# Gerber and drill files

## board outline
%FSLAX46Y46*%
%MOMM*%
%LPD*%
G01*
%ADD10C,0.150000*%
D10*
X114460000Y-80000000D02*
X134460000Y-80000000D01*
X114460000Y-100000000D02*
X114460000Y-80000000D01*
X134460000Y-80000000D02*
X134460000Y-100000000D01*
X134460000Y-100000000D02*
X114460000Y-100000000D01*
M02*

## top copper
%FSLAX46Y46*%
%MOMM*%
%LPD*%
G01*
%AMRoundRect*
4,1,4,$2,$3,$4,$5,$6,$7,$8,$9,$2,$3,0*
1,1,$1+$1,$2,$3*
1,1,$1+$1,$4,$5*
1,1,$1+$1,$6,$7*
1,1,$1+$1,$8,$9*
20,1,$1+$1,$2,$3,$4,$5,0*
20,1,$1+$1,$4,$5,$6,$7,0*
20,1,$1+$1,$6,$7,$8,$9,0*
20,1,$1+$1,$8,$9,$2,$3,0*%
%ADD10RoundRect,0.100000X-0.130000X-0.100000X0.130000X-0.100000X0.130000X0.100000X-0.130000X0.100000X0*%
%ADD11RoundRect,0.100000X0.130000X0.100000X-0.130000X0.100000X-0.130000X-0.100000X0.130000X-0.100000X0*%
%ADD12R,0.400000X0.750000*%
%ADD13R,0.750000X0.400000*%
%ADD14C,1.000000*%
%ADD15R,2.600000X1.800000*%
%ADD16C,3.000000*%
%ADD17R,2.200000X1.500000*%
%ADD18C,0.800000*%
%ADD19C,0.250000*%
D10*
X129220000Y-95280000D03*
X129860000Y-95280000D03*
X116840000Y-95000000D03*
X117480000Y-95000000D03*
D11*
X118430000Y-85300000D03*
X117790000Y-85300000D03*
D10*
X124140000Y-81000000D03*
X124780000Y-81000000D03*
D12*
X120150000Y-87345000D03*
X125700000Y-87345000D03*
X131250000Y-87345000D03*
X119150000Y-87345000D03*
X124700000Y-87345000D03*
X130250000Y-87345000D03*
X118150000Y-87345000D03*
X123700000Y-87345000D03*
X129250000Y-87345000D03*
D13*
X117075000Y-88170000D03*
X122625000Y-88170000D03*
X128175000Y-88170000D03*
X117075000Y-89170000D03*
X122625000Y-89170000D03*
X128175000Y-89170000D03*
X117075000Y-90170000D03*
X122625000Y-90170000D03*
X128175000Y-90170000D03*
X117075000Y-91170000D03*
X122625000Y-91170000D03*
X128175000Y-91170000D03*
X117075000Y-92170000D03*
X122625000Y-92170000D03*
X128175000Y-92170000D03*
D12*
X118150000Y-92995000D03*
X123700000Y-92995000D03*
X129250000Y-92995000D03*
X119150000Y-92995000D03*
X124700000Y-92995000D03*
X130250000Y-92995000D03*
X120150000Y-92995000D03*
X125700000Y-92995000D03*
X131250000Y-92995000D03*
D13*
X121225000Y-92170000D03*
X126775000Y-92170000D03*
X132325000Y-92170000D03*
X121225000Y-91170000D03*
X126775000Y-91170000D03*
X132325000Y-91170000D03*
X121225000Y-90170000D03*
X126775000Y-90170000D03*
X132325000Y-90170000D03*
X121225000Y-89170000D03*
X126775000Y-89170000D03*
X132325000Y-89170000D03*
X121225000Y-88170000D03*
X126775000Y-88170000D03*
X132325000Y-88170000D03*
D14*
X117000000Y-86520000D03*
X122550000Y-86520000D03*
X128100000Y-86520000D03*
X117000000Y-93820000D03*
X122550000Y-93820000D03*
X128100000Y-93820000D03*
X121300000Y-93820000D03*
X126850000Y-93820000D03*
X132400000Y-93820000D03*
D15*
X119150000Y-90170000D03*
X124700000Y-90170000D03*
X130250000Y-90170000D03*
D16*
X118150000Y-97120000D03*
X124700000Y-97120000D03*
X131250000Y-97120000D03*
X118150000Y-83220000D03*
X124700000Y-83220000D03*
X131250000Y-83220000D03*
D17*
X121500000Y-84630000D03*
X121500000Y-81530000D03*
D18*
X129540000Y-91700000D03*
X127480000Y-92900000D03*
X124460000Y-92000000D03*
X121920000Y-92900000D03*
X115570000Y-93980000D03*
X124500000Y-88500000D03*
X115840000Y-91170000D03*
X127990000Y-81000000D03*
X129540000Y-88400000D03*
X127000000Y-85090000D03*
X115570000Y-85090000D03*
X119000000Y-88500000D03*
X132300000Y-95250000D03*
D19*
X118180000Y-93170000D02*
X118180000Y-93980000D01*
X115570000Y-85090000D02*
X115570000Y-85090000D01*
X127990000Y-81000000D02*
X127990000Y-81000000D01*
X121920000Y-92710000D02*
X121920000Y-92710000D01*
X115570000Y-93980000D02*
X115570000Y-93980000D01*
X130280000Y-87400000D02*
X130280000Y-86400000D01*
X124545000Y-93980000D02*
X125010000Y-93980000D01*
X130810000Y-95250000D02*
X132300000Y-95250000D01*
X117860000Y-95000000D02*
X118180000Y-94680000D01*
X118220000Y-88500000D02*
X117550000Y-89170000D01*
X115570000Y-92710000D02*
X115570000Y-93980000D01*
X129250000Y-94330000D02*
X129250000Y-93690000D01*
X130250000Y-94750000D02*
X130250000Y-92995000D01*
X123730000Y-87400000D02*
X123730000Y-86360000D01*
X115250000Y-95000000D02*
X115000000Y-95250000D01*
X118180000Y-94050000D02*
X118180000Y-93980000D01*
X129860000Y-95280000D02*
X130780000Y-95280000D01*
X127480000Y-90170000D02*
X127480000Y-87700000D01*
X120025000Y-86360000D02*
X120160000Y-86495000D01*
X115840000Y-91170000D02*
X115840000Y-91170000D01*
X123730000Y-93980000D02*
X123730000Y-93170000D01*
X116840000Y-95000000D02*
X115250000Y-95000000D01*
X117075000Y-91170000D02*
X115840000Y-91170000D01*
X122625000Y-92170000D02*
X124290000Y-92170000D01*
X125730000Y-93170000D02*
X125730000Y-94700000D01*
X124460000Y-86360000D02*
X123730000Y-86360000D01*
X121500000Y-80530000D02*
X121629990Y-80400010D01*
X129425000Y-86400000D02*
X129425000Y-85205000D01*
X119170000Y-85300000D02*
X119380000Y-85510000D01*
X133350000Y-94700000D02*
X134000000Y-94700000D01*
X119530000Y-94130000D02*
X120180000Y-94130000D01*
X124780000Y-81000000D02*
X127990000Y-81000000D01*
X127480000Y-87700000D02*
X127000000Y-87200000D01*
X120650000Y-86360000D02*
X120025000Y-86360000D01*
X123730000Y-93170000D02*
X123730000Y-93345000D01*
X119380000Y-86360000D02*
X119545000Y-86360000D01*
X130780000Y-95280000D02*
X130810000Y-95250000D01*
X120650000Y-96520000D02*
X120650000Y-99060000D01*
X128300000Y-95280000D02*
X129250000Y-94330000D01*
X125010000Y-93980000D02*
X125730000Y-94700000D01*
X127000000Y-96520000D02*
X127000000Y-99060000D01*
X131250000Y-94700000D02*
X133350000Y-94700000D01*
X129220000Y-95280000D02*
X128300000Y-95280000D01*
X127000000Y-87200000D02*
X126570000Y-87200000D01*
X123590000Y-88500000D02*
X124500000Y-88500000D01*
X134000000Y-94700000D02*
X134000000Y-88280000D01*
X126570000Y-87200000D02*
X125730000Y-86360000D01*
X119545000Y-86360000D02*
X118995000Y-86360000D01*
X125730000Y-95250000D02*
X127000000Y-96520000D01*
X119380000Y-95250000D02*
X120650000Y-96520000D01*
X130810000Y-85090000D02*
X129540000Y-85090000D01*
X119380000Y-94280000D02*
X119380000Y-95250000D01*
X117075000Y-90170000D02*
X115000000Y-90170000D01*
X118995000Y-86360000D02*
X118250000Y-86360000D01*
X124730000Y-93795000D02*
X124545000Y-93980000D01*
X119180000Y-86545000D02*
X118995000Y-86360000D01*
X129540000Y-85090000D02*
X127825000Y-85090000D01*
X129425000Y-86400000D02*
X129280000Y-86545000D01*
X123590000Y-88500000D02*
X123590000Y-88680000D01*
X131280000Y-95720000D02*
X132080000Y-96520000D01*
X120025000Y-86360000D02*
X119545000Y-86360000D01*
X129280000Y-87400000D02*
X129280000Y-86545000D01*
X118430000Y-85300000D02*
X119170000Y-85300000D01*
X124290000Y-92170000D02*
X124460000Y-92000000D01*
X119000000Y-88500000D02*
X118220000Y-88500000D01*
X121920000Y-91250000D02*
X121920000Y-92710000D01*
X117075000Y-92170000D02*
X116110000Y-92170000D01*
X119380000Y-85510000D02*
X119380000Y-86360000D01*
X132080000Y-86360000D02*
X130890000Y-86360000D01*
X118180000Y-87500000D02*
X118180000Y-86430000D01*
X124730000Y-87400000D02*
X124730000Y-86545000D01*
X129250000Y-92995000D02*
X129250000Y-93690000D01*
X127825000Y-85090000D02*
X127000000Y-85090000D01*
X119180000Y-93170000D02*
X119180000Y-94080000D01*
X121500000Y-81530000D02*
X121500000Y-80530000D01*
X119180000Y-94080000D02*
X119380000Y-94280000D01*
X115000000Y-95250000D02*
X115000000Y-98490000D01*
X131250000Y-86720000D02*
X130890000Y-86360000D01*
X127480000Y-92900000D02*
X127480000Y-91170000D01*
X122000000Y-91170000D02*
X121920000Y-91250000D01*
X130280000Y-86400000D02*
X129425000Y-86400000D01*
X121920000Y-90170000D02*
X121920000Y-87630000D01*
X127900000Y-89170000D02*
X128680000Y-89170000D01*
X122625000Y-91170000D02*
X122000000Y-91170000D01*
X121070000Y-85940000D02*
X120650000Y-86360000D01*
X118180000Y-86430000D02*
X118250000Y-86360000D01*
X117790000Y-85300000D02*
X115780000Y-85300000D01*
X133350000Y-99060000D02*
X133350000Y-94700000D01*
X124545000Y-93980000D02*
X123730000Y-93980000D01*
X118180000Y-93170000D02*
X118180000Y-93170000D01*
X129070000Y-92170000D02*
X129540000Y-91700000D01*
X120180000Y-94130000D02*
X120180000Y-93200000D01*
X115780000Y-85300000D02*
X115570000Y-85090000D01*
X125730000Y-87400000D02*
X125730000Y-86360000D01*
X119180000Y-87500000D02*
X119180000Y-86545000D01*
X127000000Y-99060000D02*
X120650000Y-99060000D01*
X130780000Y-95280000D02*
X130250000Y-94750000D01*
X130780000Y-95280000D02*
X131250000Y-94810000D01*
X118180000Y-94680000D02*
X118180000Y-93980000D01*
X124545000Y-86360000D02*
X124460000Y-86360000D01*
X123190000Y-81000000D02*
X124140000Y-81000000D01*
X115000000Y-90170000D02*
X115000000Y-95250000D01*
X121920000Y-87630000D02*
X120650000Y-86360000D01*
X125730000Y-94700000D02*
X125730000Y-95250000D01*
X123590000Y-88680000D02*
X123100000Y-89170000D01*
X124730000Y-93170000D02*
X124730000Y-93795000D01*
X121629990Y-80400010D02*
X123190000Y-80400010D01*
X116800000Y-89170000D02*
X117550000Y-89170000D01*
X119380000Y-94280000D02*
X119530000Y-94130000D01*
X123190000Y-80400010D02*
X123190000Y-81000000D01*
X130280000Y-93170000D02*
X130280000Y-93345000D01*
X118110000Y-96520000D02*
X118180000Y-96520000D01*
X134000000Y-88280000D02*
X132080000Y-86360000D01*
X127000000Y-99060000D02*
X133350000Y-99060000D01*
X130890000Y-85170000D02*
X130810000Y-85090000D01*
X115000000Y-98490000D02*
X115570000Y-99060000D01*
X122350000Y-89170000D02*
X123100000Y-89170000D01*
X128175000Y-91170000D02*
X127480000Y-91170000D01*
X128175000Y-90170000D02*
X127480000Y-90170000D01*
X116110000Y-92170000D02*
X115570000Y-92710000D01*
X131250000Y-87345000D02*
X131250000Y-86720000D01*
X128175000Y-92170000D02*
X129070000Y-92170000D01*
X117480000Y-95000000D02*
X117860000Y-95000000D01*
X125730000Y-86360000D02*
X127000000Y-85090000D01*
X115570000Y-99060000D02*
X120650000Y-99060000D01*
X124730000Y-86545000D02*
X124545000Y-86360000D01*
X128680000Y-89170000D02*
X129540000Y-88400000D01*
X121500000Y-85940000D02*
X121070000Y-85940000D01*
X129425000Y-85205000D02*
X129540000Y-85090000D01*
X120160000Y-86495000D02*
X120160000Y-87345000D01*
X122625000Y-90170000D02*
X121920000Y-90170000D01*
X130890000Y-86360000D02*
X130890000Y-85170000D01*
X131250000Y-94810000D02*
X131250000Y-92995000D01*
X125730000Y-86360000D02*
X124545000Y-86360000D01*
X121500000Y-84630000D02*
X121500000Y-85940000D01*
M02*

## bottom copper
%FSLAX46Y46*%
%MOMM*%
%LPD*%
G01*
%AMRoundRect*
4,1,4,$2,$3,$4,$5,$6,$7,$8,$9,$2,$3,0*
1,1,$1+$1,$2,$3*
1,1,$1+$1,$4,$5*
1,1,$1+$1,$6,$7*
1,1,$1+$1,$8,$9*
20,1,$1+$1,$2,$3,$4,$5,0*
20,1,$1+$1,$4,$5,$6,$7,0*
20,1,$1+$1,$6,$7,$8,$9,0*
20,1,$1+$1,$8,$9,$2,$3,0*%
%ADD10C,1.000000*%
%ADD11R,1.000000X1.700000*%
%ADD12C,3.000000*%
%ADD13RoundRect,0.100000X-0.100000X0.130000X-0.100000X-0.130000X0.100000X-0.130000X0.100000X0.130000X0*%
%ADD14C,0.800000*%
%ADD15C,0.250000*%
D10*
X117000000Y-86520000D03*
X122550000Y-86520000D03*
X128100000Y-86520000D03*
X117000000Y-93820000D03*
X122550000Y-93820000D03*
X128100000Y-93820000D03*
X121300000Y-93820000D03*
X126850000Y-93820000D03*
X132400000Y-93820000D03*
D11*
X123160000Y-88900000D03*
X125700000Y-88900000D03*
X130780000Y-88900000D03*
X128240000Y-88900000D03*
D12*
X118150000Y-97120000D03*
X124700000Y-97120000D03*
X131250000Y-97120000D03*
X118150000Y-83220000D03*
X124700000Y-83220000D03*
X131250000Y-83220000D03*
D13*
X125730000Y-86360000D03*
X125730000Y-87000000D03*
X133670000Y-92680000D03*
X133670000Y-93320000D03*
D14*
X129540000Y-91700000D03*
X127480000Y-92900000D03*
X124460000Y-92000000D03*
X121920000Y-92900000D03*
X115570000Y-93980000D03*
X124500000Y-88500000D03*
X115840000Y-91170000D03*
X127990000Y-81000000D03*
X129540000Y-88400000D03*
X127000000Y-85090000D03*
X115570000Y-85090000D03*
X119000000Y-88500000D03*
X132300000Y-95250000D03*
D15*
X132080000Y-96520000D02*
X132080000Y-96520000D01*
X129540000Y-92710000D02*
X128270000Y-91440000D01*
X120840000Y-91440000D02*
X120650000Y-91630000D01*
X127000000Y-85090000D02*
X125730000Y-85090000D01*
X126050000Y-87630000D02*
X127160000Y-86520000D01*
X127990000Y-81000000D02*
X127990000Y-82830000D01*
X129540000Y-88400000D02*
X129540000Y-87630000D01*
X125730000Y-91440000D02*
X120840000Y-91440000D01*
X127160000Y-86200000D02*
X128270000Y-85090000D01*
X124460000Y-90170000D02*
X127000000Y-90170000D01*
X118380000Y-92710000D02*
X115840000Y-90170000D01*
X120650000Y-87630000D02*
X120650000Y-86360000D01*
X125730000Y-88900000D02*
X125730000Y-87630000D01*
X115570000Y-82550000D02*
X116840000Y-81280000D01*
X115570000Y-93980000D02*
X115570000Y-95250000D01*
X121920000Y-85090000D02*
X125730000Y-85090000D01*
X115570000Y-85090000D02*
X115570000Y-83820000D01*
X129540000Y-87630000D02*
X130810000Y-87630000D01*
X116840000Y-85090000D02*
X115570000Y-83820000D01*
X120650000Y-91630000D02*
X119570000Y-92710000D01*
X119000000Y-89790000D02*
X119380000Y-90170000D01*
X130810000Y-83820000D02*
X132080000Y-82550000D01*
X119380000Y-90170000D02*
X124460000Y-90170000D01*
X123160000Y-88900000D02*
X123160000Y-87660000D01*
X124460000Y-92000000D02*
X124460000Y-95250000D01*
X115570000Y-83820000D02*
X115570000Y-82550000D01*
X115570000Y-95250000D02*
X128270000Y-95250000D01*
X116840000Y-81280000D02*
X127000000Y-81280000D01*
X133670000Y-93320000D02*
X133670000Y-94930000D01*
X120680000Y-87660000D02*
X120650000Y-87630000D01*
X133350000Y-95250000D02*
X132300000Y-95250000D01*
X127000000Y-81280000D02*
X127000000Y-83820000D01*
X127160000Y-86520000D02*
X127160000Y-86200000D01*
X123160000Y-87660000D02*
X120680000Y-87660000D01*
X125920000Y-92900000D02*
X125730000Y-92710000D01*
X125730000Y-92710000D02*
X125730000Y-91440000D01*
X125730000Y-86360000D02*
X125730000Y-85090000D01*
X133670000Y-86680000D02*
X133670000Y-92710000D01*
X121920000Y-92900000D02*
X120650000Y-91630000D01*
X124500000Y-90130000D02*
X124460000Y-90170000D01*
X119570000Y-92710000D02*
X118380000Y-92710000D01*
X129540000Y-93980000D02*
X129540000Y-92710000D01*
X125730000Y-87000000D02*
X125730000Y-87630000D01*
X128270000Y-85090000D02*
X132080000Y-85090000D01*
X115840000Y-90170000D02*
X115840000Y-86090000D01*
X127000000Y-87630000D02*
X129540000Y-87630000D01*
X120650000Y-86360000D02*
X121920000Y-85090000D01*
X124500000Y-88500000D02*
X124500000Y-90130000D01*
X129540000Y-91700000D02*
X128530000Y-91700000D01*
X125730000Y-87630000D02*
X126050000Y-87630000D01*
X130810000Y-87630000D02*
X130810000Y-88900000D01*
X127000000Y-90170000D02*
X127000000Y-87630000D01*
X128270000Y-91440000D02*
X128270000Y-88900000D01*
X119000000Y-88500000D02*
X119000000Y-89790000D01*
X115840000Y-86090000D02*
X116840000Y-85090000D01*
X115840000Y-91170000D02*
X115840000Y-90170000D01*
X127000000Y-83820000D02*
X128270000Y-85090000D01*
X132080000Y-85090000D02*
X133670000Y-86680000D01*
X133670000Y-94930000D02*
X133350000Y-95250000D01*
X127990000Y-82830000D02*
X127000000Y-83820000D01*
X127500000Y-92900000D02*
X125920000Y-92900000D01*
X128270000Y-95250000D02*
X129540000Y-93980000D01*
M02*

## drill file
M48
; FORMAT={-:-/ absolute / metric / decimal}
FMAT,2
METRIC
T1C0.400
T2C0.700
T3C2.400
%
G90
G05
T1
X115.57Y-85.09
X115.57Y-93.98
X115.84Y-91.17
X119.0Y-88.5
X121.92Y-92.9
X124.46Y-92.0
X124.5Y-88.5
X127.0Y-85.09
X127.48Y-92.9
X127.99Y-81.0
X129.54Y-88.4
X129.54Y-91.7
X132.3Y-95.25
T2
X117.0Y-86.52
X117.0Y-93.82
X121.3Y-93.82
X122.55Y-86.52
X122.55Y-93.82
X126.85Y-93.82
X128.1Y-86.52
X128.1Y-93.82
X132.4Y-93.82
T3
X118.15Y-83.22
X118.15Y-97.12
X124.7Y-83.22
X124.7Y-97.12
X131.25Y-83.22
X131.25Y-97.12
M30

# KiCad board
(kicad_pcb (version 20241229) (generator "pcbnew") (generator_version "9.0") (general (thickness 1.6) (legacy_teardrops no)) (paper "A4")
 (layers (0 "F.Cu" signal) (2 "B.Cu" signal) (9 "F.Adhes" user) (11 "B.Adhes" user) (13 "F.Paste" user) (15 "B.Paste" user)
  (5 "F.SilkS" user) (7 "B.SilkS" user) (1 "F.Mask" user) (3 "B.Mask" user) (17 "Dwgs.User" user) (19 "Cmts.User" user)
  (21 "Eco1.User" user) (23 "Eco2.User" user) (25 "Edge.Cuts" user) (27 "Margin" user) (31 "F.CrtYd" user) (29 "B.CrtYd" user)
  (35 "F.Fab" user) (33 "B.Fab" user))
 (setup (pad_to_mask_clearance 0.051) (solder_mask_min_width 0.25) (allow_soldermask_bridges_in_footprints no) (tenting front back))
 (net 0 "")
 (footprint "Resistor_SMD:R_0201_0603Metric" (layer "F.Cu") (at 129.54 95.28)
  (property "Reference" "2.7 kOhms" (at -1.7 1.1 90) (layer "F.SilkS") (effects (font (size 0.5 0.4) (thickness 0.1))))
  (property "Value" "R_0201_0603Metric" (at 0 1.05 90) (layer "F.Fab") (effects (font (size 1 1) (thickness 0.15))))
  (pad "" smd roundrect (at -0.345 0) (size 0.318 0.36) (layers "F.Paste") (roundrect_rratio 0.25))
  (pad "" smd roundrect (at 0.345 0) (size 0.318 0.36) (layers "F.Paste") (roundrect_rratio 0.25))
  (pad "1" smd roundrect (at -0.32 0) (size 0.46 0.4) (layers "F.Cu" "F.Mask") (roundrect_rratio 0.25))
  (pad "2" smd roundrect (at 0.32 0) (size 0.46 0.4) (layers "F.Cu" "F.Mask") (roundrect_rratio 0.25)))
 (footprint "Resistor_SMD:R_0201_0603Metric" (layer "F.Cu") (at 117.16 95)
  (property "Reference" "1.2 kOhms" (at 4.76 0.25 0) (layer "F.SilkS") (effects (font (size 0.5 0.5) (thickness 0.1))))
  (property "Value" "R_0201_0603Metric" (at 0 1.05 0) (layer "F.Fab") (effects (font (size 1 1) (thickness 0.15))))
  (pad "" smd roundrect (at -0.345 0) (size 0.318 0.36) (layers "F.Paste") (roundrect_rratio 0.25))
  (pad "" smd roundrect (at 0.345 0) (size 0.318 0.36) (layers "F.Paste") (roundrect_rratio 0.25))
  (pad "1" smd roundrect (at -0.32 0) (size 0.46 0.4) (layers "F.Cu" "F.Mask") (roundrect_rratio 0.25))
  (pad "2" smd roundrect (at 0.32 0) (size 0.46 0.4) (layers "F.Cu" "F.Mask") (roundrect_rratio 0.25)))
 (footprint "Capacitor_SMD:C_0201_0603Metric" (layer "F.Cu") (at 118.11 85.3 180)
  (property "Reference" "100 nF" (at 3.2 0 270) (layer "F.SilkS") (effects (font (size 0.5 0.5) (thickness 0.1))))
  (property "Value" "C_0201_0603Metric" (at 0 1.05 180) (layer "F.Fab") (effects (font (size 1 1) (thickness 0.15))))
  (pad "" smd roundrect (at -0.345 0 180) (size 0.318 0.36) (layers "F.Paste") (roundrect_rratio 0.25))
  (pad "" smd roundrect (at 0.345 0 180) (size 0.318 0.36) (layers "F.Paste") (roundrect_rratio 0.25))
  (pad "1" smd roundrect (at -0.32 0 180) (size 0.46 0.4) (layers "F.Cu" "F.Mask") (roundrect_rratio 0.25))
  (pad "2" smd roundrect (at 0.32 0 180) (size 0.46 0.4) (layers "F.Cu" "F.Mask") (roundrect_rratio 0.25)))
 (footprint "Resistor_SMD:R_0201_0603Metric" (layer "F.Cu") (at 124.46 81)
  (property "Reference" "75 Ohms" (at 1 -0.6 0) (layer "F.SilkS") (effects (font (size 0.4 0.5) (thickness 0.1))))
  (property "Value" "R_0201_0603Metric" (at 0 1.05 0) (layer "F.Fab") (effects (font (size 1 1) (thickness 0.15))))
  (pad "" smd roundrect (at -0.345 0) (size 0.318 0.36) (layers "F.Paste") (roundrect_rratio 0.25))
  (pad "" smd roundrect (at 0.345 0) (size 0.318 0.36) (layers "F.Paste") (roundrect_rratio 0.25))
  (pad "1" smd roundrect (at -0.32 0) (size 0.46 0.4) (layers "F.Cu" "F.Mask") (roundrect_rratio 0.25))
  (pad "2" smd roundrect (at 0.32 0) (size 0.46 0.4) (layers "F.Cu" "F.Mask") (roundrect_rratio 0.25)))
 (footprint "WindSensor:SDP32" (layer "F.Cu") (at 124.7 90.17)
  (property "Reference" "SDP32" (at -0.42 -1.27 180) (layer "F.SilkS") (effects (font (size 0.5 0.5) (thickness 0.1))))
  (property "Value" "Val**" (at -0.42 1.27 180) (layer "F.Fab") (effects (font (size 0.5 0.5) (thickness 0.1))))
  (pad "1" smd rect (at -4.55 -2.825 270) (size 0.75 0.4) (layers "F.Cu" "F.Mask" "F.Paste"))
  (pad "1" smd rect (at 1 -2.825 270) (size 0.75 0.4) (layers "F.Cu" "F.Mask" "F.Paste"))
  (pad "1" smd rect (at 6.55 -2.825 270) (size 0.75 0.4) (layers "F.Cu" "F.Mask" "F.Paste"))
  (pad "2" smd rect (at -5.55 -2.825 270) (size 0.75 0.4) (layers "F.Cu" "F.Mask" "F.Paste"))
  (pad "2" smd rect (at 0 -2.825 270) (size 0.75 0.4) (layers "F.Cu" "F.Mask" "F.Paste"))
  (pad "2" smd rect (at 5.55 -2.825 270) (size 0.75 0.4) (layers "F.Cu" "F.Mask" "F.Paste"))
  (pad "3" smd rect (at -6.55 -2.825 270) (size 0.75 0.4) (layers "F.Cu" "F.Mask" "F.Paste"))
  (pad "3" smd rect (at -1 -2.825 270) (size 0.75 0.4) (layers "F.Cu" "F.Mask" "F.Paste"))
  (pad "3" smd rect (at 4.55 -2.825 270) (size 0.75 0.4) (layers "F.Cu" "F.Mask" "F.Paste"))
  (pad "4" smd rect (at -7.625 -2 270) (size 0.4 0.75) (layers "F.Cu" "F.Mask" "F.Paste"))
  (pad "4" smd rect (at -2.075 -2 270) (size 0.4 0.75) (layers "F.Cu" "F.Mask" "F.Paste"))
  (pad "4" smd rect (at 3.475 -2 270) (size 0.4 0.75) (layers "F.Cu" "F.Mask" "F.Paste"))
  (pad "5" smd rect (at -7.625 -1 270) (size 0.4 0.75) (layers "F.Cu" "F.Mask" "F.Paste"))
  (pad "5" smd rect (at -2.075 -1 270) (size 0.4 0.75) (layers "F.Cu" "F.Mask" "F.Paste"))
  (pad "5" smd rect (at 3.475 -1 270) (size 0.4 0.75) (layers "F.Cu" "F.Mask" "F.Paste"))
  (pad "6" smd rect (at -7.625 0 270) (size 0.4 0.75) (layers "F.Cu" "F.Mask" "F.Paste"))
  (pad "6" smd rect (at -2.075 0 270) (size 0.4 0.75) (layers "F.Cu" "F.Mask" "F.Paste"))
  (pad "6" smd rect (at 3.475 0 270) (size 0.4 0.75) (layers "F.Cu" "F.Mask" "F.Paste"))
  (pad "7" smd rect (at -7.625 1 270) (size 0.4 0.75) (layers "F.Cu" "F.Mask" "F.Paste"))
  (pad "7" smd rect (at -2.075 1 270) (size 0.4 0.75) (layers "F.Cu" "F.Mask" "F.Paste"))
  (pad "7" smd rect (at 3.475 1 270) (size 0.4 0.75) (layers "F.Cu" "F.Mask" "F.Paste"))
  (pad "8" smd rect (at -7.625 2 270) (size 0.4 0.75) (layers "F.Cu" "F.Mask" "F.Paste"))
  (pad "8" smd rect (at -2.075 2 270) (size 0.4 0.75) (layers "F.Cu" "F.Mask" "F.Paste"))
  (pad "8" smd rect (at 3.475 2 270) (size 0.4 0.75) (layers "F.Cu" "F.Mask" "F.Paste"))
  (pad "9" smd rect (at -6.55 2.825 270) (size 0.75 0.4) (layers "F.Cu" "F.Mask" "F.Paste"))
  (pad "9" smd rect (at -1 2.825 270) (size 0.75 0.4) (layers "F.Cu" "F.Mask" "F.Paste"))
  (pad "9" smd rect (at 4.55 2.825 270) (size 0.75 0.4) (layers "F.Cu" "F.Mask" "F.Paste"))
  (pad "10" smd rect (at -5.55 2.825 270) (size 0.75 0.4) (layers "F.Cu" "F.Mask" "F.Paste"))
  (pad "10" smd rect (at 0 2.825 270) (size 0.75 0.4) (layers "F.Cu" "F.Mask" "F.Paste"))
  (pad "10" smd rect (at 5.55 2.825 270) (size 0.75 0.4) (layers "F.Cu" "F.Mask" "F.Paste"))
  (pad "11" smd rect (at -4.55 2.825 270) (size 0.75 0.4) (layers "F.Cu" "F.Mask" "F.Paste"))
  (pad "11" smd rect (at 1 2.825 270) (size 0.75 0.4) (layers "F.Cu" "F.Mask" "F.Paste"))
  (pad "11" smd rect (at 6.55 2.825 270) (size 0.75 0.4) (layers "F.Cu" "F.Mask" "F.Paste"))
  (pad "12" smd rect (at -3.475 2 270) (size 0.4 0.75) (layers "F.Cu" "F.Mask" "F.Paste"))
  (pad "12" smd rect (at 2.075 2 270) (size 0.4 0.75) (layers "F.Cu" "F.Mask" "F.Paste"))
  (pad "12" smd rect (at 7.625 2 270) (size 0.4 0.75) (layers "F.Cu" "F.Mask" "F.Paste"))
  (pad "13" smd rect (at -3.475 1 270) (size 0.4 0.75) (layers "F.Cu" "F.Mask" "F.Paste"))
  (pad "13" smd rect (at 2.075 1 270) (size 0.4 0.75) (layers "F.Cu" "F.Mask" "F.Paste"))
  (pad "13" smd rect (at 7.625 1 270) (size 0.4 0.75) (layers "F.Cu" "F.Mask" "F.Paste"))
  (pad "14" smd rect (at -3.475 0 270) (size 0.4 0.75) (layers "F.Cu" "F.Mask" "F.Paste"))
  (pad "14" smd rect (at 2.075 0 270) (size 0.4 0.75) (layers "F.Cu" "F.Mask" "F.Paste"))
  (pad "14" smd rect (at 7.625 0 270) (size 0.4 0.75) (layers "F.Cu" "F.Mask" "F.Paste"))
  (pad "15" smd rect (at -3.475 -1 270) (size 0.4 0.75) (layers "F.Cu" "F.Mask" "F.Paste"))
  (pad "15" smd rect (at 2.075 -1 270) (size 0.4 0.75) (layers "F.Cu" "F.Mask" "F.Paste"))
  (pad "15" smd rect (at 7.625 -1 270) (size 0.4 0.75) (layers "F.Cu" "F.Mask" "F.Paste"))
  (pad "16" smd rect (at -3.475 -2 270) (size 0.4 0.75) (layers "F.Cu" "F.Mask" "F.Paste"))
  (pad "16" smd rect (at 2.075 -2 270) (size 0.4 0.75) (layers "F.Cu" "F.Mask" "F.Paste"))
  (pad "16" smd rect (at 7.625 -2 270) (size 0.4 0.75) (layers "F.Cu" "F.Mask" "F.Paste"))
  (pad "17" thru_hole circle (at -7.7 -3.65 270) (size 1 1) (drill 0.7) (layers "*.Cu" "*.Mask") (remove_unused_layers no))
  (pad "17" thru_hole circle (at -2.15 -3.65 270) (size 1 1) (drill 0.7) (layers "*.Cu" "*.Mask") (remove_unused_layers no))
  (pad "17" thru_hole circle (at 3.4 -3.65 270) (size 1 1) (drill 0.7) (layers "*.Cu" "*.Mask") (remove_unused_layers no))
  (pad "18" thru_hole circle (at -7.7 3.65 270) (size 1 1) (drill 0.7) (layers "*.Cu" "*.Mask") (remove_unused_layers no))
  (pad "18" thru_hole circle (at -2.15 3.65 270) (size 1 1) (drill 0.7) (layers "*.Cu" "*.Mask") (remove_unused_layers no))
  (pad "18" thru_hole circle (at 3.4 3.65 270) (size 1 1) (drill 0.7) (layers "*.Cu" "*.Mask") (remove_unused_layers no))
  (pad "19" thru_hole circle (at -3.4 3.65 270) (size 1 1) (drill 0.7) (layers "*.Cu" "*.Mask") (remove_unused_layers no))
  (pad "19" thru_hole circle (at 2.15 3.65 270) (size 1 1) (drill 0.7) (layers "*.Cu" "*.Mask") (remove_unused_layers no))
  (pad "19" thru_hole circle (at 7.7 3.65 270) (size 1 1) (drill 0.7) (layers "*.Cu" "*.Mask") (remove_unused_layers no))
  (pad "20" smd rect (at -5.55 0 270) (size 1.8 2.6) (layers "F.Cu" "F.Mask" "F.Paste"))
  (pad "20" smd rect (at 0 0 270) (size 1.8 2.6) (layers "F.Cu" "F.Mask" "F.Paste"))
  (pad "20" smd rect (at 5.55 0 270) (size 1.8 2.6) (layers "F.Cu" "F.Mask" "F.Paste"))
  (pad "21" smd rect (at -1.54 -1.27) (size 1 1.7) (layers "B.Cu" "B.Mask" "B.Paste"))
  (pad "22" smd rect (at 1 -1.27) (size 1 1.7) (layers "B.Cu" "B.Mask" "B.Paste"))
  (pad "23" smd rect (at 6.08 -1.27) (size 1 1.7) (layers "B.Cu" "B.Mask" "B.Paste"))
  (pad "24" smd rect (at 3.54 -1.27) (size 1 1.7) (layers "B.Cu" "B.Mask" "B.Paste"))
  (pad "25" thru_hole circle (at -6.55 6.95) (size 3 3) (drill 2.4) (layers "*.Cu" "*.Mask") (remove_unused_layers no))
  (pad "26" thru_hole circle (at 0 6.95) (size 3 3) (drill 2.4) (layers "*.Cu" "*.Mask") (remove_unused_layers no))
  (pad "27" thru_hole circle (at 6.55 6.95) (size 3 3) (drill 2.4) (layers "*.Cu" "*.Mask") (remove_unused_layers no))
  (pad "28" thru_hole circle (at -6.55 -6.95) (size 3 3) (drill 2.4) (layers "*.Cu" "*.Mask") (remove_unused_layers no))
  (pad "29" thru_hole circle (at 0 -6.95) (size 3 3) (drill 2.4) (layers "*.Cu" "*.Mask") (remove_unused_layers no))
  (pad "30" thru_hole circle (at 6.55 -6.95) (size 3 3) (drill 2.4) (layers "*.Cu" "*.Mask") (remove_unused_layers no)))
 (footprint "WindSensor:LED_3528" (layer "F.Cu") (at 121.5 82.8 -90)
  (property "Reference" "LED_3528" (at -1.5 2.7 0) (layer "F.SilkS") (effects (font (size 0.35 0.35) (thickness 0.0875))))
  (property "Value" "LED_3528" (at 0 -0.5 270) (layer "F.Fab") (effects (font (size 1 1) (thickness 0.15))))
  (pad "1" smd rect (at 1.83 0 270) (size 1.5 2.2) (layers "F.Cu" "F.Mask" "F.Paste"))
  (pad "2" smd rect (at -1.27 0 270) (size 1.5 2.2) (layers "F.Cu" "F.Mask" "F.Paste")))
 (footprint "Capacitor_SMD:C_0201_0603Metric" (layer "B.Cu") (at 125.73 86.68 -90)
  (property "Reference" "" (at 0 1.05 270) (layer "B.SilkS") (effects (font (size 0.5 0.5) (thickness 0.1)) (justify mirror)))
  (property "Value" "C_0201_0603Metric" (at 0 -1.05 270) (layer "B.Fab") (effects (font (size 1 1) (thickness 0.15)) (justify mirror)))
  (pad "" smd roundrect (at -0.345 0 270) (size 0.318 0.36) (layers "B.Paste") (roundrect_rratio 0.25))
  (pad "" smd roundrect (at 0.345 0 270) (size 0.318 0.36) (layers "B.Paste") (roundrect_rratio 0.25))
  (pad "1" smd roundrect (at -0.32 0 270) (size 0.46 0.4) (layers "B.Cu" "B.Mask") (roundrect_rratio 0.25))
  (pad "2" smd roundrect (at 0.32 0 270) (size 0.46 0.4) (layers "B.Cu" "B.Mask") (roundrect_rratio 0.25)))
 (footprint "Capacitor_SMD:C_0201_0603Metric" (layer "B.Cu") (at 133.67 93 -90)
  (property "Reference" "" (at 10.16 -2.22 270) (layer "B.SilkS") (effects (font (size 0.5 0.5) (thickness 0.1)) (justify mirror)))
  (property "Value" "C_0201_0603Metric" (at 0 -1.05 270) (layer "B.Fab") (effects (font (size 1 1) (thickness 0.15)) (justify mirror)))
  (pad "" smd roundrect (at -0.345 0 270) (size 0.318 0.36) (layers "B.Paste") (roundrect_rratio 0.25))
  (pad "" smd roundrect (at 0.345 0 270) (size 0.318 0.36) (layers "B.Paste") (roundrect_rratio 0.25))
  (pad "1" smd roundrect (at -0.32 0 270) (size 0.46 0.4) (layers "B.Cu" "B.Mask") (roundrect_rratio 0.25))
  (pad "2" smd roundrect (at 0.32 0 270) (size 0.46 0.4) (layers "B.Cu" "B.Mask") (roundrect_rratio 0.25)))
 (gr_line (start 114.46 80) (end 134.46 80) (stroke (width 0.15) (type solid)) (layer "Edge.Cuts"))
 (gr_line (start 114.46 100) (end 114.46 80) (stroke (width 0.15) (type solid)) (layer "Edge.Cuts"))
 (gr_line (start 134.46 80) (end 134.46 100) (stroke (width 0.15) (type solid)) (layer "Edge.Cuts"))
 (gr_line (start 134.46 100) (end 114.46 100) (stroke (width 0.15) (type solid)) (layer "Edge.Cuts"))
 (segment (start 118.18 93.17) (end 118.18 93.98) (width 0.25) (layer "F.Cu") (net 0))
 (segment (start 115.57 85.09) (end 115.57 85.09) (width 0.25) (layer "F.Cu") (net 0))
 (segment (start 127.99 81) (end 127.99 81) (width 0.25) (layer "F.Cu") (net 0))
 (segment (start 121.92 92.71) (end 121.92 92.71) (width 0.25) (layer "F.Cu") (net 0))
 (segment (start 115.57 93.98) (end 115.57 93.98) (width 0.25) (layer "F.Cu") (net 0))
 (segment (start 130.28 87.4) (end 130.28 86.4) (width 0.25) (layer "F.Cu") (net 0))
 (segment (start 124.545 93.98) (end 125.01 93.98) (width 0.25) (layer "F.Cu") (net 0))
 (segment (start 130.81 95.25) (end 132.3 95.25) (width 0.25) (layer "F.Cu") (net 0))
 (segment (start 117.86 95) (end 118.18 94.68) (width 0.25) (layer "F.Cu") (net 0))
 (segment (start 118.22 88.5) (end 117.55 89.17) (width 0.25) (layer "F.Cu") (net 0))
 (segment (start 115.57 92.71) (end 115.57 93.98) (width 0.25) (layer "F.Cu") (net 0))
 (segment (start 129.25 94.33) (end 129.25 93.69) (width 0.25) (layer "F.Cu") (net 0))
 (segment (start 130.25 94.75) (end 130.25 92.995) (width 0.25) (layer "F.Cu") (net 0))
 (segment (start 123.73 87.4) (end 123.73 86.36) (width 0.25) (layer "F.Cu") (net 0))
 (segment (start 115.25 95) (end 115 95.25) (width 0.25) (layer "F.Cu") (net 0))
 (segment (start 118.18 94.05) (end 118.18 93.98) (width 0.25) (layer "F.Cu") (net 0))
 (segment (start 129.86 95.28) (end 130.78 95.28) (width 0.25) (layer "F.Cu") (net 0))
 (segment (start 127.48 90.17) (end 127.48 87.7) (width 0.25) (layer "F.Cu") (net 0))
 (segment (start 120.025 86.36) (end 120.16 86.495) (width 0.25) (layer "F.Cu") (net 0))
 (segment (start 115.84 91.17) (end 115.84 91.17) (width 0.25) (layer "F.Cu") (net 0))
 (segment (start 123.73 93.98) (end 123.73 93.17) (width 0.25) (layer "F.Cu") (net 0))
 (segment (start 116.84 95) (end 115.25 95) (width 0.25) (layer "F.Cu") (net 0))
 (segment (start 117.075 91.17) (end 115.84 91.17) (width 0.25) (layer "F.Cu") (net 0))
 (segment (start 122.625 92.17) (end 124.29 92.17) (width 0.25) (layer "F.Cu") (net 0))
 (segment (start 125.73 93.17) (end 125.73 94.7) (width 0.25) (layer "F.Cu") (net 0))
 (segment (start 124.46 86.36) (end 123.73 86.36) (width 0.25) (layer "F.Cu") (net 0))
 (segment (start 121.5 80.53) (end 121.62999 80.40001) (width 0.25) (layer "F.Cu") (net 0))
 (segment (start 129.425 86.4) (end 129.425 85.205) (width 0.25) (layer "F.Cu") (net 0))
 (segment (start 119.17 85.3) (end 119.38 85.51) (width 0.25) (layer "F.Cu") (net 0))
 (segment (start 133.35 94.7) (end 134 94.7) (width 0.25) (layer "F.Cu") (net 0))
 (segment (start 119.53 94.13) (end 120.18 94.13) (width 0.25) (layer "F.Cu") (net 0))
 (segment (start 124.78 81) (end 127.99 81) (width 0.25) (layer "F.Cu") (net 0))
 (segment (start 127.48 87.7) (end 127 87.2) (width 0.25) (layer "F.Cu") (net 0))
 (segment (start 120.65 86.36) (end 120.025 86.36) (width 0.25) (layer "F.Cu") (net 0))
 (segment (start 123.73 93.17) (end 123.73 93.345) (width 0.25) (layer "F.Cu") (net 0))
 (segment (start 119.38 86.36) (end 119.545 86.36) (width 0.25) (layer "F.Cu") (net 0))
 (segment (start 130.78 95.28) (end 130.81 95.25) (width 0.25) (layer "F.Cu") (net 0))
 (segment (start 120.65 96.52) (end 120.65 99.06) (width 0.25) (layer "F.Cu") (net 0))
 (segment (start 128.3 95.28) (end 129.25 94.33) (width 0.25) (layer "F.Cu") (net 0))
 (segment (start 125.01 93.98) (end 125.73 94.7) (width 0.25) (layer "F.Cu") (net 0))
 (segment (start 127 96.52) (end 127 99.06) (width 0.25) (layer "F.Cu") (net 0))
 (segment (start 131.25 94.7) (end 133.35 94.7) (width 0.25) (layer "F.Cu") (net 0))
 (segment (start 129.22 95.28) (end 128.3 95.28) (width 0.25) (layer "F.Cu") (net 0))
 (segment (start 127 87.2) (end 126.57 87.2) (width 0.25) (layer "F.Cu") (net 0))
 (segment (start 123.59 88.5) (end 124.5 88.5) (width 0.25) (layer "F.Cu") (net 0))
 (segment (start 134 94.7) (end 134 88.28) (width 0.25) (layer "F.Cu") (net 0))
 (segment (start 126.57 87.2) (end 125.73 86.36) (width 0.25) (layer "F.Cu") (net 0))
 (segment (start 119.545 86.36) (end 118.995 86.36) (width 0.25) (layer "F.Cu") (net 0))
 (segment (start 125.73 95.25) (end 127 96.52) (width 0.25) (layer "F.Cu") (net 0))
 (segment (start 119.38 95.25) (end 120.65 96.52) (width 0.25) (layer "F.Cu") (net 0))
 (segment (start 130.81 85.09) (end 129.54 85.09) (width 0.25) (layer "F.Cu") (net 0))
 (segment (start 119.38 94.28) (end 119.38 95.25) (width 0.25) (layer "F.Cu") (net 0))
 (segment (start 117.075 90.17) (end 115 90.17) (width 0.25) (layer "F.Cu") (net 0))
 (segment (start 118.995 86.36) (end 118.25 86.36) (width 0.25) (layer "F.Cu") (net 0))
 (segment (start 124.73 93.795) (end 124.545 93.98) (width 0.25) (layer "F.Cu") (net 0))
 (segment (start 119.18 86.545) (end 118.995 86.36) (width 0.25) (layer "F.Cu") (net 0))
 (segment (start 129.54 85.09) (end 127.825 85.09) (width 0.25) (layer "F.Cu") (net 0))
 (segment (start 129.425 86.4) (end 129.28 86.545) (width 0.25) (layer "F.Cu") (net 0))
 (segment (start 123.59 88.5) (end 123.59 88.68) (width 0.25) (layer "F.Cu") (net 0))
 (segment (start 131.28 95.72) (end 132.08 96.52) (width 0.25) (layer "F.Cu") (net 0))
 (segment (start 120.025 86.36) (end 119.545 86.36) (width 0.25) (layer "F.Cu") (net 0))
 (segment (start 129.28 87.4) (end 129.28 86.545) (width 0.25) (layer "F.Cu") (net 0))
 (segment (start 118.43 85.3) (end 119.17 85.3) (width 0.25) (layer "F.Cu") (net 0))
 (segment (start 124.29 92.17) (end 124.46 92) (width 0.25) (layer "F.Cu") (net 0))
 (segment (start 119 88.5) (end 118.22 88.5) (width 0.25) (layer "F.Cu") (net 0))
 (segment (start 121.92 91.25) (end 121.92 92.71) (width 0.25) (layer "F.Cu") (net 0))
 (segment (start 117.075 92.17) (end 116.11 92.17) (width 0.25) (layer "F.Cu") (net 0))
 (segment (start 119.38 85.51) (end 119.38 86.36) (width 0.25) (layer "F.Cu") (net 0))
 (segment (start 132.08 86.36) (end 130.89 86.36) (width 0.25) (layer "F.Cu") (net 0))
 (segment (start 118.18 87.5) (end 118.18 86.43) (width 0.25) (layer "F.Cu") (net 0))
 (segment (start 124.73 87.4) (end 124.73 86.545) (width 0.25) (layer "F.Cu") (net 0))
 (segment (start 129.25 92.995) (end 129.25 93.69) (width 0.25) (layer "F.Cu") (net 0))
 (segment (start 127.825 85.09) (end 127 85.09) (width 0.25) (layer "F.Cu") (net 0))
 (segment (start 119.18 93.17) (end 119.18 94.08) (width 0.25) (layer "F.Cu") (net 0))
 (segment (start 121.5 81.53) (end 121.5 80.53) (width 0.25) (layer "F.Cu") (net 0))
 (segment (start 119.18 94.08) (end 119.38 94.28) (width 0.25) (layer "F.Cu") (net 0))
 (segment (start 115 95.25) (end 115 98.49) (width 0.25) (layer "F.Cu") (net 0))
 (segment (start 131.25 86.72) (end 130.89 86.36) (width 0.25) (layer "F.Cu") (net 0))
 (segment (start 127.48 92.9) (end 127.48 91.17) (width 0.25) (layer "F.Cu") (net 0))
 (segment (start 122 91.17) (end 121.92 91.25) (width 0.25) (layer "F.Cu") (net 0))
 (segment (start 130.28 86.4) (end 129.425 86.4) (width 0.25) (layer "F.Cu") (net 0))
 (segment (start 121.92 90.17) (end 121.92 87.63) (width 0.25) (layer "F.Cu") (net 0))
 (segment (start 127.9 89.17) (end 128.68 89.17) (width 0.25) (layer "F.Cu") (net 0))
 (segment (start 122.625 91.17) (end 122 91.17) (width 0.25) (layer "F.Cu") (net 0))
 (segment (start 121.07 85.94) (end 120.65 86.36) (width 0.25) (layer "F.Cu") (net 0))
 (segment (start 118.18 86.43) (end 118.25 86.36) (width 0.25) (layer "F.Cu") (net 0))
 (segment (start 117.79 85.3) (end 115.78 85.3) (width 0.25) (layer "F.Cu") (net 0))
 (segment (start 133.35 99.06) (end 133.35 94.7) (width 0.25) (layer "F.Cu") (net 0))
 (segment (start 124.545 93.98) (end 123.73 93.98) (width 0.25) (layer "F.Cu") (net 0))
 (segment (start 118.18 93.17) (end 118.18 93.17) (width 0.25) (layer "F.Cu") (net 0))
 (segment (start 129.07 92.17) (end 129.54 91.7) (width 0.25) (layer "F.Cu") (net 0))
 (segment (start 120.18 94.13) (end 120.18 93.2) (width 0.25) (layer "F.Cu") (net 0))
 (segment (start 115.78 85.3) (end 115.57 85.09) (width 0.25) (layer "F.Cu") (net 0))
 (segment (start 125.73 87.4) (end 125.73 86.36) (width 0.25) (layer "F.Cu") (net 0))
 (segment (start 119.18 87.5) (end 119.18 86.545) (width 0.25) (layer "F.Cu") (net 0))
 (segment (start 127 99.06) (end 120.65 99.06) (width 0.25) (layer "F.Cu") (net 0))
 (segment (start 130.78 95.28) (end 130.25 94.75) (width 0.25) (layer "F.Cu") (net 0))
 (segment (start 130.78 95.28) (end 131.25 94.81) (width 0.25) (layer "F.Cu") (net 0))
 (segment (start 118.18 94.68) (end 118.18 93.98) (width 0.25) (layer "F.Cu") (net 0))
 (segment (start 124.545 86.36) (end 124.46 86.36) (width 0.25) (layer "F.Cu") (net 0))
 (segment (start 123.19 81) (end 124.14 81) (width 0.25) (layer "F.Cu") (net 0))
 (segment (start 115 90.17) (end 115 95.25) (width 0.25) (layer "F.Cu") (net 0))
 (segment (start 121.92 87.63) (end 120.65 86.36) (width 0.25) (layer "F.Cu") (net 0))
 (segment (start 125.73 94.7) (end 125.73 95.25) (width 0.25) (layer "F.Cu") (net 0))
 (segment (start 123.59 88.68) (end 123.1 89.17) (width 0.25) (layer "F.Cu") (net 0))
 (segment (start 124.73 93.17) (end 124.73 93.795) (width 0.25) (layer "F.Cu") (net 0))
 (segment (start 121.62999 80.40001) (end 123.19 80.40001) (width 0.25) (layer "F.Cu") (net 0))
 (segment (start 116.8 89.17) (end 117.55 89.17) (width 0.25) (layer "F.Cu") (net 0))
 (segment (start 119.38 94.28) (end 119.53 94.13) (width 0.25) (layer "F.Cu") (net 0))
 (segment (start 123.19 80.40001) (end 123.19 81) (width 0.25) (layer "F.Cu") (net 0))
 (segment (start 130.28 93.17) (end 130.28 93.345) (width 0.25) (layer "F.Cu") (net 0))
 (segment (start 118.11 96.52) (end 118.18 96.52) (width 0.25) (layer "F.Cu") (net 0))
 (segment (start 134 88.28) (end 132.08 86.36) (width 0.25) (layer "F.Cu") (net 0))
 (segment (start 127 99.06) (end 133.35 99.06) (width 0.25) (layer "F.Cu") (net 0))
 (segment (start 130.89 85.17) (end 130.81 85.09) (width 0.25) (layer "F.Cu") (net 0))
 (segment (start 115 98.49) (end 115.57 99.06) (width 0.25) (layer "F.Cu") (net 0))
 (segment (start 122.35 89.17) (end 123.1 89.17) (width 0.25) (layer "F.Cu") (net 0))
 (segment (start 128.175 91.17) (end 127.48 91.17) (width 0.25) (layer "F.Cu") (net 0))
 (segment (start 128.175 90.17) (end 127.48 90.17) (width 0.25) (layer "F.Cu") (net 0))
 (segment (start 116.11 92.17) (end 115.57 92.71) (width 0.25) (layer "F.Cu") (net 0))
 (segment (start 131.25 87.345) (end 131.25 86.72) (width 0.25) (layer "F.Cu") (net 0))
 (segment (start 128.175 92.17) (end 129.07 92.17) (width 0.25) (layer "F.Cu") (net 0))
 (segment (start 117.48 95) (end 117.86 95) (width 0.25) (layer "F.Cu") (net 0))
 (segment (start 125.73 86.36) (end 127 85.09) (width 0.25) (layer "F.Cu") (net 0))
 (segment (start 115.57 99.06) (end 120.65 99.06) (width 0.25) (layer "F.Cu") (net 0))
 (segment (start 124.73 86.545) (end 124.545 86.36) (width 0.25) (layer "F.Cu") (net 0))
 (segment (start 128.68 89.17) (end 129.54 88.4) (width 0.25) (layer "F.Cu") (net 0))
 (segment (start 121.5 85.94) (end 121.07 85.94) (width 0.25) (layer "F.Cu") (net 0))
 (segment (start 129.425 85.205) (end 129.54 85.09) (width 0.25) (layer "F.Cu") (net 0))
 (segment (start 120.16 86.495) (end 120.16 87.345) (width 0.25) (layer "F.Cu") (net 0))
 (segment (start 122.625 90.17) (end 121.92 90.17) (width 0.25) (layer "F.Cu") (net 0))
 (segment (start 130.89 86.36) (end 130.89 85.17) (width 0.25) (layer "F.Cu") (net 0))
 (segment (start 131.25 94.81) (end 131.25 92.995) (width 0.25) (layer "F.Cu") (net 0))
 (segment (start 125.73 86.36) (end 124.545 86.36) (width 0.25) (layer "F.Cu") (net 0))
 (segment (start 121.5 84.63) (end 121.5 85.94) (width 0.25) (layer "F.Cu") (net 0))
 (via (at 129.54 91.7) (size 0.8) (drill 0.4) (layers "F.Cu" "B.Cu") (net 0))
 (via (at 127.48 92.9) (size 0.8) (drill 0.4) (layers "F.Cu" "B.Cu") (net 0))
 (via (at 124.46 92) (size 0.8) (drill 0.4) (layers "F.Cu" "B.Cu") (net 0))
 (via (at 121.92 92.9) (size 0.8) (drill 0.4) (layers "F.Cu" "B.Cu") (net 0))
 (via (at 115.57 93.98) (size 0.8) (drill 0.4) (layers "F.Cu" "B.Cu") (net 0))
 (via (at 124.5 88.5) (size 0.8) (drill 0.4) (layers "F.Cu" "B.Cu") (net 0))
 (via (at 115.84 91.17) (size 0.8) (drill 0.4) (layers "F.Cu" "B.Cu") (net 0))
 (via (at 127.99 81) (size 0.8) (drill 0.4) (layers "F.Cu" "B.Cu") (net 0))
 (via (at 129.54 88.4) (size 0.8) (drill 0.4) (layers "F.Cu" "B.Cu") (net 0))
 (via (at 127 85.09) (size 0.8) (drill 0.4) (layers "F.Cu" "B.Cu") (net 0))
 (via (at 115.57 85.09) (size 0.8) (drill 0.4) (layers "F.Cu" "B.Cu") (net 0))
 (via (at 119 88.5) (size 0.8) (drill 0.4) (layers "F.Cu" "B.Cu") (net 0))
 (via (at 132.3 95.25) (size 0.8) (drill 0.4) (layers "F.Cu" "B.Cu") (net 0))
 (segment (start 132.08 96.52) (end 132.08 96.52) (width 0.25) (layer "B.Cu") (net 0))
 (segment (start 129.54 92.71) (end 128.27 91.44) (width 0.25) (layer "B.Cu") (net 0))
 (segment (start 120.84 91.44) (end 120.65 91.63) (width 0.25) (layer "B.Cu") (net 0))
 (segment (start 127 85.09) (end 125.73 85.09) (width 0.25) (layer "B.Cu") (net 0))
 (segment (start 126.05 87.63) (end 127.16 86.52) (width 0.25) (layer "B.Cu") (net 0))
 (segment (start 127.99 81) (end 127.99 82.83) (width 0.25) (layer "B.Cu") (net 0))
 (segment (start 129.54 88.4) (end 129.54 87.63) (width 0.25) (layer "B.Cu") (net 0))
 (segment (start 125.73 91.44) (end 120.84 91.44) (width 0.25) (layer "B.Cu") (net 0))
 (segment (start 127.16 86.2) (end 128.27 85.09) (width 0.25) (layer "B.Cu") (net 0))
 (segment (start 124.46 90.17) (end 127 90.17) (width 0.25) (layer "B.Cu") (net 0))
 (segment (start 118.38 92.71) (end 115.84 90.17) (width 0.25) (layer "B.Cu") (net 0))
 (segment (start 120.65 87.63) (end 120.65 86.36) (width 0.25) (layer "B.Cu") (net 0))
 (segment (start 125.73 88.9) (end 125.73 87.63) (width 0.25) (layer "B.Cu") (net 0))
 (segment (start 115.57 82.55) (end 116.84 81.28) (width 0.25) (layer "B.Cu") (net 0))
 (segment (start 115.57 93.98) (end 115.57 95.25) (width 0.25) (layer "B.Cu") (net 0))
 (segment (start 121.92 85.09) (end 125.73 85.09) (width 0.25) (layer "B.Cu") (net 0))
 (segment (start 115.57 85.09) (end 115.57 83.82) (width 0.25) (layer "B.Cu") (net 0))
 (segment (start 129.54 87.63) (end 130.81 87.63) (width 0.25) (layer "B.Cu") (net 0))
 (segment (start 116.84 85.09) (end 115.57 83.82) (width 0.25) (layer "B.Cu") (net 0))
 (segment (start 120.65 91.63) (end 119.57 92.71) (width 0.25) (layer "B.Cu") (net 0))
 (segment (start 119 89.79) (end 119.38 90.17) (width 0.25) (layer "B.Cu") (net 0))
 (segment (start 130.81 83.82) (end 132.08 82.55) (width 0.25) (layer "B.Cu") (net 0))
 (segment (start 119.38 90.17) (end 124.46 90.17) (width 0.25) (layer "B.Cu") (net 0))
 (segment (start 123.16 88.9) (end 123.16 87.66) (width 0.25) (layer "B.Cu") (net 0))
 (segment (start 124.46 92) (end 124.46 95.25) (width 0.25) (layer "B.Cu") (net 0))
 (segment (start 115.57 83.82) (end 115.57 82.55) (width 0.25) (layer "B.Cu") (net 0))
 (segment (start 115.57 95.25) (end 128.27 95.25) (width 0.25) (layer "B.Cu") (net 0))
 (segment (start 116.84 81.28) (end 127 81.28) (width 0.25) (layer "B.Cu") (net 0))
 (segment (start 133.67 93.32) (end 133.67 94.93) (width 0.25) (layer "B.Cu") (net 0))
 (segment (start 120.68 87.66) (end 120.65 87.63) (width 0.25) (layer "B.Cu") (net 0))
 (segment (start 133.35 95.25) (end 132.3 95.25) (width 0.25) (layer "B.Cu") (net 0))
 (segment (start 127 81.28) (end 127 83.82) (width 0.25) (layer "B.Cu") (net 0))
 (segment (start 127.16 86.52) (end 127.16 86.2) (width 0.25) (layer "B.Cu") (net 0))
 (segment (start 123.16 87.66) (end 120.68 87.66) (width 0.25) (layer "B.Cu") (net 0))
 (segment (start 125.92 92.9) (end 125.73 92.71) (width 0.25) (layer "B.Cu") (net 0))
 (segment (start 125.73 92.71) (end 125.73 91.44) (width 0.25) (layer "B.Cu") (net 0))
 (segment (start 125.73 86.36) (end 125.73 85.09) (width 0.25) (layer "B.Cu") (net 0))
 (segment (start 133.67 86.68) (end 133.67 92.71) (width 0.25) (layer "B.Cu") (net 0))
 (segment (start 121.92 92.9) (end 120.65 91.63) (width 0.25) (layer "B.Cu") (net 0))
 (segment (start 124.5 90.13) (end 124.46 90.17) (width 0.25) (layer "B.Cu") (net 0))
 (segment (start 119.57 92.71) (end 118.38 92.71) (width 0.25) (layer "B.Cu") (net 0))
 (segment (start 129.54 93.98) (end 129.54 92.71) (width 0.25) (layer "B.Cu") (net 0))
 (segment (start 125.73 87) (end 125.73 87.63) (width 0.25) (layer "B.Cu") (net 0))
 (segment (start 128.27 85.09) (end 132.08 85.09) (width 0.25) (layer "B.Cu") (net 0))
 (segment (start 115.84 90.17) (end 115.84 86.09) (width 0.25) (layer "B.Cu") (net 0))
 (segment (start 127 87.63) (end 129.54 87.63) (width 0.25) (layer "B.Cu") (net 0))
 (segment (start 120.65 86.36) (end 121.92 85.09) (width 0.25) (layer "B.Cu") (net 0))
 (segment (start 124.5 88.5) (end 124.5 90.13) (width 0.25) (layer "B.Cu") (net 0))
 (segment (start 129.54 91.7) (end 128.53 91.7) (width 0.25) (layer "B.Cu") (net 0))
 (segment (start 125.73 87.63) (end 126.05 87.63) (width 0.25) (layer "B.Cu") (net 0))
 (segment (start 130.81 87.63) (end 130.81 88.9) (width 0.25) (layer "B.Cu") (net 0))
 (segment (start 127 90.17) (end 127 87.63) (width 0.25) (layer "B.Cu") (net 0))
 (segment (start 128.27 91.44) (end 128.27 88.9) (width 0.25) (layer "B.Cu") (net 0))
 (segment (start 119 88.5) (end 119 89.79) (width 0.25) (layer "B.Cu") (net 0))
 (segment (start 115.84 86.09) (end 116.84 85.09) (width 0.25) (layer "B.Cu") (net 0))
 (segment (start 115.84 91.17) (end 115.84 90.17) (width 0.25) (layer "B.Cu") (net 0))
 (segment (start 127 83.82) (end 128.27 85.09) (width 0.25) (layer "B.Cu") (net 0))
 (segment (start 132.08 85.09) (end 133.67 86.68) (width 0.25) (layer "B.Cu") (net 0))
 (segment (start 133.67 94.93) (end 133.35 95.25) (width 0.25) (layer "B.Cu") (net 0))
 (segment (start 127.99 82.83) (end 127 83.82) (width 0.25) (layer "B.Cu") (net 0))
 (segment (start 127.5 92.9) (end 125.92 92.9) (width 0.25) (layer "B.Cu") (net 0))
 (segment (start 128.27 95.25) (end 129.54 93.98) (width 0.25) (layer "B.Cu") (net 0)))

